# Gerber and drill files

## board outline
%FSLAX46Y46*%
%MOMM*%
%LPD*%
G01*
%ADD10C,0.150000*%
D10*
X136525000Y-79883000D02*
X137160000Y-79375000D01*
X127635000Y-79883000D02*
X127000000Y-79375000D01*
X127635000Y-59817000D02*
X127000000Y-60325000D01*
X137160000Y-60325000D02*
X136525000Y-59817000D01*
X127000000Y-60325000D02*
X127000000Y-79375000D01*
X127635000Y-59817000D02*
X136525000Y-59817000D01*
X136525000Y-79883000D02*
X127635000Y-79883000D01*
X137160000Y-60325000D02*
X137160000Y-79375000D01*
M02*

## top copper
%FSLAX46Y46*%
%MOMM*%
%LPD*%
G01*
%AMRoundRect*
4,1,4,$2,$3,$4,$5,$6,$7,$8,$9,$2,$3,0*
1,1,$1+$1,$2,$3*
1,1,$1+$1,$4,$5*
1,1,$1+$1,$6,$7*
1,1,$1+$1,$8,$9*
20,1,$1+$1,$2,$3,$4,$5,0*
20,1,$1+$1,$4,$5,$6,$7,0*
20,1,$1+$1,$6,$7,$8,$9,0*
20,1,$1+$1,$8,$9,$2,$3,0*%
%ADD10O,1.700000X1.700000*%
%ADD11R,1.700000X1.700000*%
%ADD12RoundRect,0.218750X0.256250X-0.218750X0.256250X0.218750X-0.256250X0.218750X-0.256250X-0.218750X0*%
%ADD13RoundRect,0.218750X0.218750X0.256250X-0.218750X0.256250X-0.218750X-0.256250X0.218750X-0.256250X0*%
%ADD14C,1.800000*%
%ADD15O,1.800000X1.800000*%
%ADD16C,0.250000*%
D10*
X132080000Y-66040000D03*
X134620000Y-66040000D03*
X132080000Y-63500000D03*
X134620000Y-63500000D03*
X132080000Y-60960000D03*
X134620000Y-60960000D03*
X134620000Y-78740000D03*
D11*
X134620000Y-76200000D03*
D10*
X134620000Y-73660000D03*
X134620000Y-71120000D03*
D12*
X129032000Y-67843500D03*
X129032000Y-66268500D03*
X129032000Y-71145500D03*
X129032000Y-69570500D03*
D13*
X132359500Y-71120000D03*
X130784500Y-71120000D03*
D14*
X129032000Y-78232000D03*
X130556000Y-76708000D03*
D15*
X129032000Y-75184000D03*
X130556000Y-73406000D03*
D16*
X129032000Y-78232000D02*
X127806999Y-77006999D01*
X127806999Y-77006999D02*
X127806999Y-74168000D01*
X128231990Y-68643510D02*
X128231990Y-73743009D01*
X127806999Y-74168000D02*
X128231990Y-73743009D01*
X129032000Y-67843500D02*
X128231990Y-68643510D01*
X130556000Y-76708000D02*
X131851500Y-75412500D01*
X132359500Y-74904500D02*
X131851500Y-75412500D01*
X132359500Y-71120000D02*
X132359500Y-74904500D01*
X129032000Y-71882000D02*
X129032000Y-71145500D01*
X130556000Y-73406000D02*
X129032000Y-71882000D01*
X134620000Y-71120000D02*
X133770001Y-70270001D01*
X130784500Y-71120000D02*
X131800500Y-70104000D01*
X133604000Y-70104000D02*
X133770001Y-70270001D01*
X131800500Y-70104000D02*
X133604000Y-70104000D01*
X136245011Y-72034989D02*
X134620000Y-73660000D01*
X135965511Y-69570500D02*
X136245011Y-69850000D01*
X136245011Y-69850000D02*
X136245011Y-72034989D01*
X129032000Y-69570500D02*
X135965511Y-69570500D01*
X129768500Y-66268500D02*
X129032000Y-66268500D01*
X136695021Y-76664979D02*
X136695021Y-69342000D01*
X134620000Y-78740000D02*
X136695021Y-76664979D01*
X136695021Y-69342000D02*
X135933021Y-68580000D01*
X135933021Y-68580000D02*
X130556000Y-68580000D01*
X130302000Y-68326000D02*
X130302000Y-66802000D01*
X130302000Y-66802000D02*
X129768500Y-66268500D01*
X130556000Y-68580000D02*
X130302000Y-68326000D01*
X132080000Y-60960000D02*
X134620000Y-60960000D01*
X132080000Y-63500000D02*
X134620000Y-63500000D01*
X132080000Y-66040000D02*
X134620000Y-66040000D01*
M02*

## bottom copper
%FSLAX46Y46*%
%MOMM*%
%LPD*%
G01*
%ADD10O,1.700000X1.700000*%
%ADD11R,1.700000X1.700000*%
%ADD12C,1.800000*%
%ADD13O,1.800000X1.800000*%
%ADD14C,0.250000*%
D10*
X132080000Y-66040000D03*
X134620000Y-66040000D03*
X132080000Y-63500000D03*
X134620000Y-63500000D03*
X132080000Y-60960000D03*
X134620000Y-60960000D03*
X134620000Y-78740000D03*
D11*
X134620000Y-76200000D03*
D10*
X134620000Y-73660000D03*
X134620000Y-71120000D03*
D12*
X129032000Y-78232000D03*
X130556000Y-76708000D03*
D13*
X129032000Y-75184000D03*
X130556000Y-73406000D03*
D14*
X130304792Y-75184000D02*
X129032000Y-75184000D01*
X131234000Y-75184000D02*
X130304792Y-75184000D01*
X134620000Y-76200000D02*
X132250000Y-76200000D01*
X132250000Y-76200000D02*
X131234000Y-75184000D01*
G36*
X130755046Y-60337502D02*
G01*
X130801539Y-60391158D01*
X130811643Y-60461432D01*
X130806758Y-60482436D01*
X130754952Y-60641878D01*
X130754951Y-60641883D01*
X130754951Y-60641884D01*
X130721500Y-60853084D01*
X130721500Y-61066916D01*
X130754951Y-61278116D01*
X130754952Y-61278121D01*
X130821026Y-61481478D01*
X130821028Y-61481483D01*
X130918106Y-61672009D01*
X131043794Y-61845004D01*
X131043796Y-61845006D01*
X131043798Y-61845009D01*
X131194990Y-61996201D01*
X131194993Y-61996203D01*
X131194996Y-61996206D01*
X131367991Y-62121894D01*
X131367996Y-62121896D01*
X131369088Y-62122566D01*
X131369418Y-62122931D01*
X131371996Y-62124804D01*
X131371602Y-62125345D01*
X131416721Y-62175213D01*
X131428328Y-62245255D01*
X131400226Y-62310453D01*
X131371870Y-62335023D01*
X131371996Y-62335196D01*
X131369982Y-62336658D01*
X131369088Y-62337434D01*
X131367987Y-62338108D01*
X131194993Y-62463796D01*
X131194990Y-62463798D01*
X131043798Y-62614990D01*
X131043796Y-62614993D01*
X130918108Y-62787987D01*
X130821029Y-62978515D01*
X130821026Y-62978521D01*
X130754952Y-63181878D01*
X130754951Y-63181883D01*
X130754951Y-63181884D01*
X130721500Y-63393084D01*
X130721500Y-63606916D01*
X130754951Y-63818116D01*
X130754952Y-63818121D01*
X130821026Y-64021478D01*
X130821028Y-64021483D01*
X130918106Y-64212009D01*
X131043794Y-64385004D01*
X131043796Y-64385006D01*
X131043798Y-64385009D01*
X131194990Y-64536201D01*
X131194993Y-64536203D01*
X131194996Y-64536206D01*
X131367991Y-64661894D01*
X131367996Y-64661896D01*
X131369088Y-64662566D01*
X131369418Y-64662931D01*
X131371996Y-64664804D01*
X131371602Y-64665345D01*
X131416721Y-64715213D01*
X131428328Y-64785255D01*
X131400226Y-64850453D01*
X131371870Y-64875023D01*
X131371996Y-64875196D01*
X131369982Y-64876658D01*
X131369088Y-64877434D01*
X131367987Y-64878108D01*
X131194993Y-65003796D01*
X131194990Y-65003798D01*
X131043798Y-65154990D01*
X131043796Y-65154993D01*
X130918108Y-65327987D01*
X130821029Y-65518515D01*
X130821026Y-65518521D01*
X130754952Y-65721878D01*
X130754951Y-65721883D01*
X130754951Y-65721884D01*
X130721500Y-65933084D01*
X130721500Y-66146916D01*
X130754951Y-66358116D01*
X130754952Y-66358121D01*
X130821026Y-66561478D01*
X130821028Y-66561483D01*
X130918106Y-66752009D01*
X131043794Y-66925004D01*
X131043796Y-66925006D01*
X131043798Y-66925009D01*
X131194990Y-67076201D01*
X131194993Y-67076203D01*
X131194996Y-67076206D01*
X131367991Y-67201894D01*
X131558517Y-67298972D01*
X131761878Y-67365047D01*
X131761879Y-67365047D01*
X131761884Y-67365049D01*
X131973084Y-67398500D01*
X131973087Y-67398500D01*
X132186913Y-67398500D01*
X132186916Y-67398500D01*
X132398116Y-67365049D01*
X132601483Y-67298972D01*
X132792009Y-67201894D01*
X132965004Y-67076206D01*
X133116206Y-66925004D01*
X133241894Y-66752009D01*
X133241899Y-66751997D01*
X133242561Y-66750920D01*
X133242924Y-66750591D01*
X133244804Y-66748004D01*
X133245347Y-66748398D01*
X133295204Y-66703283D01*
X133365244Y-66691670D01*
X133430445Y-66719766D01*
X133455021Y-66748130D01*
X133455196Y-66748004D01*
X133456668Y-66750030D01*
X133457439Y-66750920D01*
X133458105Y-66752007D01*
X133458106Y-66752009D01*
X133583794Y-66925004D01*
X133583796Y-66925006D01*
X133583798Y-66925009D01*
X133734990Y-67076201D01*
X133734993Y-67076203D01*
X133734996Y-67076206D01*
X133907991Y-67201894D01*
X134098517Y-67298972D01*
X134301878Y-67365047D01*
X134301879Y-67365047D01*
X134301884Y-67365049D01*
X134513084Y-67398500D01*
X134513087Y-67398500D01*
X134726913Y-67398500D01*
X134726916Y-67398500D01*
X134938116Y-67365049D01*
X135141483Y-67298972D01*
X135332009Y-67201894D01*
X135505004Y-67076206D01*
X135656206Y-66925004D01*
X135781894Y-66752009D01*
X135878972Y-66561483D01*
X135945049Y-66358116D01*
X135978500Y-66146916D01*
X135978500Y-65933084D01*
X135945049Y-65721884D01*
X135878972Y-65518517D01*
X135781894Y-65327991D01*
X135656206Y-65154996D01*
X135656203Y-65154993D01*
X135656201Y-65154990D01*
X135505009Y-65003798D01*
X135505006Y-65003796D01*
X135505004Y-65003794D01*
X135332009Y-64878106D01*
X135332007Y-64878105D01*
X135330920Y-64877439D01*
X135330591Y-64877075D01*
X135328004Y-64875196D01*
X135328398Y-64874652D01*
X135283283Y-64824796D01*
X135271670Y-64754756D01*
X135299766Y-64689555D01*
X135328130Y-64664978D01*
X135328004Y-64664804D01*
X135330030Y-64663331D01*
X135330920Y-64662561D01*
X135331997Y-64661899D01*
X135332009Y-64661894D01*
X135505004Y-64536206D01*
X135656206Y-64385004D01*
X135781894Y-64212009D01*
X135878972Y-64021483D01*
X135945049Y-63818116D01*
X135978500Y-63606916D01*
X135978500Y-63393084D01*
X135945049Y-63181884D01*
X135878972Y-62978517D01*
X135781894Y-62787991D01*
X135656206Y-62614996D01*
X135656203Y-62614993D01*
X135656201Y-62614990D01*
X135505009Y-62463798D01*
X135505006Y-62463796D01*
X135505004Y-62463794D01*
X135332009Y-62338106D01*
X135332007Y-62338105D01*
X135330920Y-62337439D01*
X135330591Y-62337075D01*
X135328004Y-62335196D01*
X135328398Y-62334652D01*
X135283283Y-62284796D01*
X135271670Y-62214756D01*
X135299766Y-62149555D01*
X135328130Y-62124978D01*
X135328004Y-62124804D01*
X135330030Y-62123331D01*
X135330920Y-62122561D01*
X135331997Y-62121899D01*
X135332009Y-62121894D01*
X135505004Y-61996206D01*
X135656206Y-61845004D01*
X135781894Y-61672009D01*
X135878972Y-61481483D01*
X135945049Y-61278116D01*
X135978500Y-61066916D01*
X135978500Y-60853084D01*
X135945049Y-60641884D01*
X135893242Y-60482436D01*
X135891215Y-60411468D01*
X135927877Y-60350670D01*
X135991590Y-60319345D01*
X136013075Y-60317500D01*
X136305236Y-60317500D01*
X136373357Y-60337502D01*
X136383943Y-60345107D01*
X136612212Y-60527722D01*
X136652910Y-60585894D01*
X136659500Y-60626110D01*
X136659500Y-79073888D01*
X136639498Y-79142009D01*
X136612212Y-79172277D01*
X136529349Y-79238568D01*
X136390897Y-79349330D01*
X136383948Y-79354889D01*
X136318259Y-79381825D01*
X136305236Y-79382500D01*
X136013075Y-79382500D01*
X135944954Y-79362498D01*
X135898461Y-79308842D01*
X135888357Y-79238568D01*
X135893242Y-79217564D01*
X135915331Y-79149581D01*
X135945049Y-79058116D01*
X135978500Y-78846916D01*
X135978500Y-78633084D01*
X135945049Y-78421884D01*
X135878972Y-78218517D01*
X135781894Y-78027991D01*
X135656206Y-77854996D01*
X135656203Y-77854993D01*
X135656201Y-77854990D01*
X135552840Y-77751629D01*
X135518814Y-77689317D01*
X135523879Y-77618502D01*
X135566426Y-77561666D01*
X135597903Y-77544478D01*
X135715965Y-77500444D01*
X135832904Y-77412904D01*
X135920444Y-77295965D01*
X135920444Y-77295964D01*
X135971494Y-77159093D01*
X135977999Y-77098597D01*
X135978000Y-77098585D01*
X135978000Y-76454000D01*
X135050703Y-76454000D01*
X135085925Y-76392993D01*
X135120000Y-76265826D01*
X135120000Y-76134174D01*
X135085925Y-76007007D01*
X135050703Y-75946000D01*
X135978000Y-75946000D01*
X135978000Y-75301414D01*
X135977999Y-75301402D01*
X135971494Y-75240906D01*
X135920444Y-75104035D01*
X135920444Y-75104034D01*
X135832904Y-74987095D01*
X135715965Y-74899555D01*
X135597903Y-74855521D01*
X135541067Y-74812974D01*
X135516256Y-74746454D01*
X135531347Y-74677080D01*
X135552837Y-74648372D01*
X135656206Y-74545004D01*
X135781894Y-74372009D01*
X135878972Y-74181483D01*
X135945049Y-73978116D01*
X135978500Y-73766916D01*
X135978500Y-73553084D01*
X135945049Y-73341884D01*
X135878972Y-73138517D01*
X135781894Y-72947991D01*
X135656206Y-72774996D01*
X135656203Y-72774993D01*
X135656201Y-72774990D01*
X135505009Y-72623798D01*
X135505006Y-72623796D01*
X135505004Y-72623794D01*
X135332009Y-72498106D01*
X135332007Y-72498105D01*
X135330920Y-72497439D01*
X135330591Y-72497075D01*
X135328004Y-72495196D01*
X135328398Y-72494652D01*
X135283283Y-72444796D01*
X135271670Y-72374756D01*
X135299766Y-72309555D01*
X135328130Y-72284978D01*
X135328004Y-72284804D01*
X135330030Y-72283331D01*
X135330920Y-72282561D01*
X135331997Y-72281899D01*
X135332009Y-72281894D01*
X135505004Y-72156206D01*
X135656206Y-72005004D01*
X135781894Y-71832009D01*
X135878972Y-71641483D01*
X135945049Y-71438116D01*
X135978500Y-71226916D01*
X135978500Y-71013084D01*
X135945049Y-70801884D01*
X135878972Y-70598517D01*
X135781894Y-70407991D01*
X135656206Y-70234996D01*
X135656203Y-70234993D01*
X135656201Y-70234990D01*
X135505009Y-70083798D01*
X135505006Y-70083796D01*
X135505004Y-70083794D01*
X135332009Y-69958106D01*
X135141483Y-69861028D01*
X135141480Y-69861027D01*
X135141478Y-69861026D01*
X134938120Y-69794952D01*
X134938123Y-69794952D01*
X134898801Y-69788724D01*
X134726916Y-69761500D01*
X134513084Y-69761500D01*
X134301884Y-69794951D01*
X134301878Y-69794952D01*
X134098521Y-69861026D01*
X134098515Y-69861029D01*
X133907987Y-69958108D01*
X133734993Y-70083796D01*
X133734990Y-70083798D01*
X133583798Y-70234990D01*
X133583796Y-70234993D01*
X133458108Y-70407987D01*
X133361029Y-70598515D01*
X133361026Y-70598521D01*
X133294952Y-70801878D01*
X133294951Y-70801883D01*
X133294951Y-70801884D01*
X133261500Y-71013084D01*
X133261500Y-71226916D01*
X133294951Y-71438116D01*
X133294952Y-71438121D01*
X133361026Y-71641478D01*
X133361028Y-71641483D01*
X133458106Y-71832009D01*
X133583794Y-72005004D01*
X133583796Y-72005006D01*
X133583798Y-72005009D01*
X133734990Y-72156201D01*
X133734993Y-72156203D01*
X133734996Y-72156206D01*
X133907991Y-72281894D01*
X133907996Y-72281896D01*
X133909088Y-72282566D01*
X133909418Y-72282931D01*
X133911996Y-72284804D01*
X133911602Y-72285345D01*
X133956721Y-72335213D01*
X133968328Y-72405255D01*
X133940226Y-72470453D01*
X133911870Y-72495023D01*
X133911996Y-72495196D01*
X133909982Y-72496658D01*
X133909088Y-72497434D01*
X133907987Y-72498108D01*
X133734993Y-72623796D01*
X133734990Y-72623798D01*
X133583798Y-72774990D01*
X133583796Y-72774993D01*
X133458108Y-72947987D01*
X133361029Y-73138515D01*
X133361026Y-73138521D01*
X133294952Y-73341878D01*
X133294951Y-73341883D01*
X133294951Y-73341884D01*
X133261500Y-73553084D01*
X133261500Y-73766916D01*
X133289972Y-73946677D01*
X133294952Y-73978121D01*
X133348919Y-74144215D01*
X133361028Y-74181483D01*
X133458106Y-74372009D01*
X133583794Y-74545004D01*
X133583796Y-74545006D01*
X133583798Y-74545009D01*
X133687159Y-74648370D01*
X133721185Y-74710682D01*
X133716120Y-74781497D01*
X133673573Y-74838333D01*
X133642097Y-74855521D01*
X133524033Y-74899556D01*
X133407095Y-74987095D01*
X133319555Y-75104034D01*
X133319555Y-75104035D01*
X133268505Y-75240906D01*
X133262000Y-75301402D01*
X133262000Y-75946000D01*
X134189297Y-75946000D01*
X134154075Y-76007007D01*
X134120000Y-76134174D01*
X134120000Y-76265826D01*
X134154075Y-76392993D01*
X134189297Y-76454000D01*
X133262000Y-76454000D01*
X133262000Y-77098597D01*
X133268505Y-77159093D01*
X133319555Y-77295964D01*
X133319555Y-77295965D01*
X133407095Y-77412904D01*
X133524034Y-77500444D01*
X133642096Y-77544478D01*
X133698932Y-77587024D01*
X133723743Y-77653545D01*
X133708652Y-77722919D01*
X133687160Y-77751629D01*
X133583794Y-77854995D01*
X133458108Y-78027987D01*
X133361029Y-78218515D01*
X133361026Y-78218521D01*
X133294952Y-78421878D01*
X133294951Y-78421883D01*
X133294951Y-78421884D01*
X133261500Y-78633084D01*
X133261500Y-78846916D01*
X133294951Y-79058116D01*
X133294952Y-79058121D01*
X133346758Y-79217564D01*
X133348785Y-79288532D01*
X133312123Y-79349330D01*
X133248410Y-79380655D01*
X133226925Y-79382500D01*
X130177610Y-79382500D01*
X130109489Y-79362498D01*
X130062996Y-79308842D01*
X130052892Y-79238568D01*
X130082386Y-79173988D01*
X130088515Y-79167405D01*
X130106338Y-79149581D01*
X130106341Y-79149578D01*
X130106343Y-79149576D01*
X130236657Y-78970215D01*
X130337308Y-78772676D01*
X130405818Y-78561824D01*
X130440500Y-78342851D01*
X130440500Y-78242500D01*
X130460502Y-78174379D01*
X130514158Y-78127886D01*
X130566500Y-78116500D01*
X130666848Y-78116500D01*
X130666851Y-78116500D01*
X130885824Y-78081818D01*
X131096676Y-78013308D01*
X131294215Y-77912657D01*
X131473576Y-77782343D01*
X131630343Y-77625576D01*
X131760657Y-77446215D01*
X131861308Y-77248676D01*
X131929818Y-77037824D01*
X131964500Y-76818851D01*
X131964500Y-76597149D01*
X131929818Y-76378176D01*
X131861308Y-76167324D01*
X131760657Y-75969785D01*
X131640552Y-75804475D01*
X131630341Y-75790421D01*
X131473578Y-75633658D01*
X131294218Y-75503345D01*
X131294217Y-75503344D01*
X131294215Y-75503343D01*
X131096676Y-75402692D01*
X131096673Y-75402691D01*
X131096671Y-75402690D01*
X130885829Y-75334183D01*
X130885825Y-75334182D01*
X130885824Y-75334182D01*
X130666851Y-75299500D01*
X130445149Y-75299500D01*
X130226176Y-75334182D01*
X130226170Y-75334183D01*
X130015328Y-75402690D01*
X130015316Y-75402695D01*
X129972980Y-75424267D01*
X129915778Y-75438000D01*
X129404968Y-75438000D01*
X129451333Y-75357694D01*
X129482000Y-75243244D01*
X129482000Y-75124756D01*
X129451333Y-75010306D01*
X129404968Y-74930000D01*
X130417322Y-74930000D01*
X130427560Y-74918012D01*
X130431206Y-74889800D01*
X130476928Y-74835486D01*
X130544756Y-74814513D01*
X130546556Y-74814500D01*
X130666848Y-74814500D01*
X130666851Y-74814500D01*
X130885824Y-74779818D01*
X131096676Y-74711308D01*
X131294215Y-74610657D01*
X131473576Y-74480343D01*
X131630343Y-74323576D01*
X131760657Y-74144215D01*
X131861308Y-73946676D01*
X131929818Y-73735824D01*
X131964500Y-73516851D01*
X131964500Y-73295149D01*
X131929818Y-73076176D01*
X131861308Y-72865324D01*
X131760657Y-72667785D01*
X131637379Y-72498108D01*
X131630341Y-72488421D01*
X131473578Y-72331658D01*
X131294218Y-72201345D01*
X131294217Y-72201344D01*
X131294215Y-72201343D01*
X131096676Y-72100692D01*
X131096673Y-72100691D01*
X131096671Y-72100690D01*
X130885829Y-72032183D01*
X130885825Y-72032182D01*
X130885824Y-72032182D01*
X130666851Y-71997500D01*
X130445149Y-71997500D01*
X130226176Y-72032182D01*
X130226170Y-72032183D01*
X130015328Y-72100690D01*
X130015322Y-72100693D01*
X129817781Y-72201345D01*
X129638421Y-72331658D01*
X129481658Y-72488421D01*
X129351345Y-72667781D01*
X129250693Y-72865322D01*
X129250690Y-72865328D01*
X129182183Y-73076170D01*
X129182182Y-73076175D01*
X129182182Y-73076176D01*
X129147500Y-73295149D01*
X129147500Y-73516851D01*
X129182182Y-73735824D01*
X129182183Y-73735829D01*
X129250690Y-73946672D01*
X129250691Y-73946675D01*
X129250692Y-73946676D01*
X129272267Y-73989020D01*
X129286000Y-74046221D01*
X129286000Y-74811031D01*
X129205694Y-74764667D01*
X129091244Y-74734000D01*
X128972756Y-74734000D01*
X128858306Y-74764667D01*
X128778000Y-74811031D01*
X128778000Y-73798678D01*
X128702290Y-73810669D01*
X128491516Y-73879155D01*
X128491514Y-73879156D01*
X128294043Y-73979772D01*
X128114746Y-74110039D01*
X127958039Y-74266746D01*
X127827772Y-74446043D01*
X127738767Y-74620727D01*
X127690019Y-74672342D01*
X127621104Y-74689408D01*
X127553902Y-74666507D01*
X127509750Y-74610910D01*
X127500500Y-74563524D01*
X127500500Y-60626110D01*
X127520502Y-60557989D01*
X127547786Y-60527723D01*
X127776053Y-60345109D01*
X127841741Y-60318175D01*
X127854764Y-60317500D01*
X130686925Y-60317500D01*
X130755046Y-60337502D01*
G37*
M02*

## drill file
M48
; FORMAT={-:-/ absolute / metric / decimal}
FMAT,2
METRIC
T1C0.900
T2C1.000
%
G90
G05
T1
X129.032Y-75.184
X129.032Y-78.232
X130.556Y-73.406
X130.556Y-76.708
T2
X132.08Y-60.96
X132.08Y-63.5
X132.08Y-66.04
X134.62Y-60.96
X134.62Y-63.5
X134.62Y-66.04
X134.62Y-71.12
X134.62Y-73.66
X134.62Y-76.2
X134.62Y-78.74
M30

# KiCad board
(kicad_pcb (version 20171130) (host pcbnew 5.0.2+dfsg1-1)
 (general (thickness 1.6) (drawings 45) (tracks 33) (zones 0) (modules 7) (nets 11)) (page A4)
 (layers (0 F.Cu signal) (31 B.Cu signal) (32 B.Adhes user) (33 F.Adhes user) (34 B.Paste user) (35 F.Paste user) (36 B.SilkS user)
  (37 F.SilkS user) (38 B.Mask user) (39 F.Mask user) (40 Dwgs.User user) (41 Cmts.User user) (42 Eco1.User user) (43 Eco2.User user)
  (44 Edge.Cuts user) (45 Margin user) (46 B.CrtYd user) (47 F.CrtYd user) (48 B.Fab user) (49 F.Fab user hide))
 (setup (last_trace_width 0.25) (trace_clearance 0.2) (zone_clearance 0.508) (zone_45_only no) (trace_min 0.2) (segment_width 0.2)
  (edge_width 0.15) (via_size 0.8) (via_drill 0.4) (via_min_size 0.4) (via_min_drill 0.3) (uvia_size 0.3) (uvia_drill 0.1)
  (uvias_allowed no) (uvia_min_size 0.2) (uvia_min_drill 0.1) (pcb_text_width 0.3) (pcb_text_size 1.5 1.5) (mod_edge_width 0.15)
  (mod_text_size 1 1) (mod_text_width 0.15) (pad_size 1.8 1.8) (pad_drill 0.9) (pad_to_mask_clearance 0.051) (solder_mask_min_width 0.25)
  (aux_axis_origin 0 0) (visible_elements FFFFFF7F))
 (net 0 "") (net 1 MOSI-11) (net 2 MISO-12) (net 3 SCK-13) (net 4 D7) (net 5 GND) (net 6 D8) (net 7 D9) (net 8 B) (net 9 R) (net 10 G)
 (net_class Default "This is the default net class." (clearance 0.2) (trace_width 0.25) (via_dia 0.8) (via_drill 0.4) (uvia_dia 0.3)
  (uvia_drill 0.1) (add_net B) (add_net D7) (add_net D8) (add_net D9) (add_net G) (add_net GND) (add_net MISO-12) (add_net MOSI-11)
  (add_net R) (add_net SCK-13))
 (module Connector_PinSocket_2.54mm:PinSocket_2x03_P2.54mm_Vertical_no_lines (layer F.Cu) (at 134.62 60.96)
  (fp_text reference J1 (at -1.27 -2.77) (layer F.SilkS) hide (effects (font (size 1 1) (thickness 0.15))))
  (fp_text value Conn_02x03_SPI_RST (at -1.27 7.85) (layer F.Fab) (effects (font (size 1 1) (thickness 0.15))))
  (pad 6 thru_hole oval (at -2.54 5.08) (size 1.7 1.7) (drill 1) (layers *.Cu *.Mask) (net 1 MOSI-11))
  (pad 5 thru_hole oval (at 0 5.08) (size 1.7 1.7) (drill 1) (layers *.Cu *.Mask) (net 1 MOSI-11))
  (pad 4 thru_hole oval (at -2.54 2.54) (size 1.7 1.7) (drill 1) (layers *.Cu *.Mask) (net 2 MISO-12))
  (pad 3 thru_hole oval (at 0 2.54) (size 1.7 1.7) (drill 1) (layers *.Cu *.Mask) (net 2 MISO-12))
  (pad 2 thru_hole oval (at -2.54 0) (size 1.7 1.7) (drill 1) (layers *.Cu *.Mask) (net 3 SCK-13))
  (pad 1 thru_hole oval (at 0 0) (size 1.7 1.7) (drill 1) (layers *.Cu *.Mask) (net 3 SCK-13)))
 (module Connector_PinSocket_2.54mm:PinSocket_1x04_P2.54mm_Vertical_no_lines (layer F.Cu) (at 134.62 71.12)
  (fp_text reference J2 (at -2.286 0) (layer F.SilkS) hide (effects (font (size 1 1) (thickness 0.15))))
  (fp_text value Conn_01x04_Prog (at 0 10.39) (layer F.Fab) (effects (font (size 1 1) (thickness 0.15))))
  (pad 4 thru_hole oval (at 0 7.62) (size 1.7 1.7) (drill 1) (layers *.Cu *.Mask) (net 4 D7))
  (pad 3 thru_hole rect (at 0 5.08) (size 1.7 1.7) (drill 1) (layers *.Cu *.Mask) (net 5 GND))
  (pad 2 thru_hole oval (at 0 2.54) (size 1.7 1.7) (drill 1) (layers *.Cu *.Mask) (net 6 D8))
  (pad 1 thru_hole oval (at 0 0) (size 1.7 1.7) (drill 1) (layers *.Cu *.Mask) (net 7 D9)))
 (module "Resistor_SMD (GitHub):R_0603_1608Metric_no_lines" (layer F.Cu) (at 129.032 67.056 90)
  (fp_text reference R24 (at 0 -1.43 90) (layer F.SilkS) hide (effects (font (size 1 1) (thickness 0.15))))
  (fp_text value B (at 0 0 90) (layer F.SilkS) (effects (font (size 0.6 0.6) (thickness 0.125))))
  (pad 1 smd roundrect (at -0.7875 0 90) (size 0.875 0.95) (layers F.Cu F.Paste F.Mask) (roundrect_rratio 0.25) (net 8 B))
  (pad 2 smd roundrect (at 0.7875 0 90) (size 0.875 0.95) (layers F.Cu F.Paste F.Mask) (roundrect_rratio 0.25) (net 4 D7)))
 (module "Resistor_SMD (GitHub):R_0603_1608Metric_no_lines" (layer F.Cu) (at 129.032 70.358 90)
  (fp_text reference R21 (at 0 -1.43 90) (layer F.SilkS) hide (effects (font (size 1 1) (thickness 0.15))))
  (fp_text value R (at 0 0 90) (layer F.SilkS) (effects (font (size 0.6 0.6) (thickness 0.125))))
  (pad 1 smd roundrect (at -0.7875 0 90) (size 0.875 0.95) (layers F.Cu F.Paste F.Mask) (roundrect_rratio 0.25) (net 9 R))
  (pad 2 smd roundrect (at 0.7875 0 90) (size 0.875 0.95) (layers F.Cu F.Paste F.Mask) (roundrect_rratio 0.25) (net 6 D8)))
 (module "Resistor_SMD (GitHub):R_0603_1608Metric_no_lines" (layer F.Cu) (at 131.572 71.12 180)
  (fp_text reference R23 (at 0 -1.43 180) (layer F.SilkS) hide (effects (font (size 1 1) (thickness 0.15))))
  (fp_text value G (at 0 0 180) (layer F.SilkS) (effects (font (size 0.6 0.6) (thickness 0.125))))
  (pad 1 smd roundrect (at -0.7875 0 180) (size 0.875 0.95) (layers F.Cu F.Paste F.Mask) (roundrect_rratio 0.25) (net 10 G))
  (pad 2 smd roundrect (at 0.7875 0 180) (size 0.875 0.95) (layers F.Cu F.Paste F.Mask) (roundrect_rratio 0.25) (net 7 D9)))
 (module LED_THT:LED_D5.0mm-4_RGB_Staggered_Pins (layer F.Cu) (at 130.556 73.406 270)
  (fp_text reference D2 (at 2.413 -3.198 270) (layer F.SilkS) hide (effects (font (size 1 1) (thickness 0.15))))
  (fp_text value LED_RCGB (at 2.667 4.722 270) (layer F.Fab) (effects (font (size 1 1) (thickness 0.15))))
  (pad 4 thru_hole circle (at 4.826 1.524 270) (size 1.8 1.8) (drill 0.9) (layers *.Cu *.Mask) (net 8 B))
  (pad 3 thru_hole circle (at 3.302 0 270) (size 1.8 1.8) (drill 0.9) (layers *.Cu *.Mask) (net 10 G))
  (pad 2 thru_hole oval (at 1.778 1.524 270) (size 1.8 1.8) (drill 0.9) (layers *.Cu *.Mask) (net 5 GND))
  (pad 1 thru_hole oval (at 0 0 270) (size 1.8 1.8) (drill 0.9) (layers *.Cu *.Mask) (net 9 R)))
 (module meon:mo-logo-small (layer F.Cu) (at 128.524 62.738 90)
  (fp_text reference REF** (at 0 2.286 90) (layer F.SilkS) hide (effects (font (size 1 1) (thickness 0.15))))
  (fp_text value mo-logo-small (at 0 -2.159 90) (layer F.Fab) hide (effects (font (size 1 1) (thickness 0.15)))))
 (gr_line (start 136.525 79.883) (end 137.16 79.375) (layer Edge.Cuts) (width 0.15))
 (gr_line (start 127.635 79.883) (end 127 79.375) (layer Edge.Cuts) (width 0.15))
 (gr_line (start 127.635 59.817) (end 127 60.325) (layer Edge.Cuts) (width 0.15))
 (gr_line (start 137.16 60.325) (end 136.525 59.817) (layer Edge.Cuts) (width 0.15))
 (gr_line (start 127 60.325) (end 127 79.375) (layer Edge.Cuts) (width 0.15))
 (gr_line (start 127.635 59.817) (end 136.525 59.817) (layer Edge.Cuts) (width 0.15))
 (gr_line (start 136.525 79.883) (end 127.635 79.883) (layer Edge.Cuts) (width 0.15))
 (gr_line (start 137.16 60.325) (end 137.16 79.375) (layer Edge.Cuts) (width 0.15))
 (segment (start 129.032 78.232) (end 127.806999 77.006999) (width 0.25) (layer F.Cu) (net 8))
 (segment (start 127.806999 77.006999) (end 127.806999 74.168) (width 0.25) (layer F.Cu) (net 8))
 (segment (start 128.23199 68.64351) (end 128.23199 73.743009) (width 0.25) (layer F.Cu) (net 8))
 (segment (start 127.806999 74.168) (end 128.23199 73.743009) (width 0.25) (layer F.Cu) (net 8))
 (segment (start 129.032 67.8435) (end 128.23199 68.64351) (width 0.25) (layer F.Cu) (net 8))
 (segment (start 130.556 76.708) (end 131.8515 75.4125) (width 0.25) (layer F.Cu) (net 10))
 (segment (start 132.3595 74.9045) (end 131.8515 75.4125) (width 0.25) (layer F.Cu) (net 10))
 (segment (start 132.3595 71.12) (end 132.3595 74.9045) (width 0.25) (layer F.Cu) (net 10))
 (segment (start 130.304792 75.184) (end 129.032 75.184) (width 0.25) (layer B.Cu) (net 5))
 (segment (start 131.234 75.184) (end 130.304792 75.184) (width 0.25) (layer B.Cu) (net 5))
 (segment (start 134.62 76.2) (end 132.25 76.2) (width 0.25) (layer B.Cu) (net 5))
 (segment (start 132.25 76.2) (end 131.234 75.184) (width 0.25) (layer B.Cu) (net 5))
 (segment (start 129.032 71.882) (end 129.032 71.1455) (width 0.25) (layer F.Cu) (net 9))
 (segment (start 130.556 73.406) (end 129.032 71.882) (width 0.25) (layer F.Cu) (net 9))
 (segment (start 134.62 71.12) (end 133.770001 70.270001) (width 0.25) (layer F.Cu) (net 7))
 (segment (start 130.7845 71.12) (end 131.8005 70.104) (width 0.25) (layer F.Cu) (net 7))
 (segment (start 133.604 70.104) (end 133.770001 70.270001) (width 0.25) (layer F.Cu) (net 7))
 (segment (start 131.8005 70.104) (end 133.604 70.104) (width 0.25) (layer F.Cu) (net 7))
 (segment (start 136.245011 72.034989) (end 134.62 73.66) (width 0.25) (layer F.Cu) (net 6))
 (segment (start 135.965511 69.5705) (end 136.245011 69.85) (width 0.25) (layer F.Cu) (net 6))
 (segment (start 136.245011 69.85) (end 136.245011 72.034989) (width 0.25) (layer F.Cu) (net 6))
 (segment (start 129.032 69.5705) (end 135.965511 69.5705) (width 0.25) (layer F.Cu) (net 6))
 (segment (start 129.7685 66.2685) (end 129.032 66.2685) (width 0.25) (layer F.Cu) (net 4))
 (segment (start 136.695021 76.664979) (end 136.695021 69.342) (width 0.25) (layer F.Cu) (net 4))
 (segment (start 134.62 78.74) (end 136.695021 76.664979) (width 0.25) (layer F.Cu) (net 4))
 (segment (start 136.695021 69.342) (end 135.933021 68.58) (width 0.25) (layer F.Cu) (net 4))
 (segment (start 135.933021 68.58) (end 130.556 68.58) (width 0.25) (layer F.Cu) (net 4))
 (segment (start 130.302 68.326) (end 130.302 66.802) (width 0.25) (layer F.Cu) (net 4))
 (segment (start 130.302 66.802) (end 129.7685 66.2685) (width 0.25) (layer F.Cu) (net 4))
 (segment (start 130.556 68.58) (end 130.302 68.326) (width 0.25) (layer F.Cu) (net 4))
 (segment (start 132.08 60.96) (end 134.62 60.96) (width 0.25) (layer F.Cu) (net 3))
 (segment (start 132.08 63.5) (end 134.62 63.5) (width 0.25) (layer F.Cu) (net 2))
 (segment (start 132.08 66.04) (end 134.62 66.04) (width 0.25) (layer F.Cu) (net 1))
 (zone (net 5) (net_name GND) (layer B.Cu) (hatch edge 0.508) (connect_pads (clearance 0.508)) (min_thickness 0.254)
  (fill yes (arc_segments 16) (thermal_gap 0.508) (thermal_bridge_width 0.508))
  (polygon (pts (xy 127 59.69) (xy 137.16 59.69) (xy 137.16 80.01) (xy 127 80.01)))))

